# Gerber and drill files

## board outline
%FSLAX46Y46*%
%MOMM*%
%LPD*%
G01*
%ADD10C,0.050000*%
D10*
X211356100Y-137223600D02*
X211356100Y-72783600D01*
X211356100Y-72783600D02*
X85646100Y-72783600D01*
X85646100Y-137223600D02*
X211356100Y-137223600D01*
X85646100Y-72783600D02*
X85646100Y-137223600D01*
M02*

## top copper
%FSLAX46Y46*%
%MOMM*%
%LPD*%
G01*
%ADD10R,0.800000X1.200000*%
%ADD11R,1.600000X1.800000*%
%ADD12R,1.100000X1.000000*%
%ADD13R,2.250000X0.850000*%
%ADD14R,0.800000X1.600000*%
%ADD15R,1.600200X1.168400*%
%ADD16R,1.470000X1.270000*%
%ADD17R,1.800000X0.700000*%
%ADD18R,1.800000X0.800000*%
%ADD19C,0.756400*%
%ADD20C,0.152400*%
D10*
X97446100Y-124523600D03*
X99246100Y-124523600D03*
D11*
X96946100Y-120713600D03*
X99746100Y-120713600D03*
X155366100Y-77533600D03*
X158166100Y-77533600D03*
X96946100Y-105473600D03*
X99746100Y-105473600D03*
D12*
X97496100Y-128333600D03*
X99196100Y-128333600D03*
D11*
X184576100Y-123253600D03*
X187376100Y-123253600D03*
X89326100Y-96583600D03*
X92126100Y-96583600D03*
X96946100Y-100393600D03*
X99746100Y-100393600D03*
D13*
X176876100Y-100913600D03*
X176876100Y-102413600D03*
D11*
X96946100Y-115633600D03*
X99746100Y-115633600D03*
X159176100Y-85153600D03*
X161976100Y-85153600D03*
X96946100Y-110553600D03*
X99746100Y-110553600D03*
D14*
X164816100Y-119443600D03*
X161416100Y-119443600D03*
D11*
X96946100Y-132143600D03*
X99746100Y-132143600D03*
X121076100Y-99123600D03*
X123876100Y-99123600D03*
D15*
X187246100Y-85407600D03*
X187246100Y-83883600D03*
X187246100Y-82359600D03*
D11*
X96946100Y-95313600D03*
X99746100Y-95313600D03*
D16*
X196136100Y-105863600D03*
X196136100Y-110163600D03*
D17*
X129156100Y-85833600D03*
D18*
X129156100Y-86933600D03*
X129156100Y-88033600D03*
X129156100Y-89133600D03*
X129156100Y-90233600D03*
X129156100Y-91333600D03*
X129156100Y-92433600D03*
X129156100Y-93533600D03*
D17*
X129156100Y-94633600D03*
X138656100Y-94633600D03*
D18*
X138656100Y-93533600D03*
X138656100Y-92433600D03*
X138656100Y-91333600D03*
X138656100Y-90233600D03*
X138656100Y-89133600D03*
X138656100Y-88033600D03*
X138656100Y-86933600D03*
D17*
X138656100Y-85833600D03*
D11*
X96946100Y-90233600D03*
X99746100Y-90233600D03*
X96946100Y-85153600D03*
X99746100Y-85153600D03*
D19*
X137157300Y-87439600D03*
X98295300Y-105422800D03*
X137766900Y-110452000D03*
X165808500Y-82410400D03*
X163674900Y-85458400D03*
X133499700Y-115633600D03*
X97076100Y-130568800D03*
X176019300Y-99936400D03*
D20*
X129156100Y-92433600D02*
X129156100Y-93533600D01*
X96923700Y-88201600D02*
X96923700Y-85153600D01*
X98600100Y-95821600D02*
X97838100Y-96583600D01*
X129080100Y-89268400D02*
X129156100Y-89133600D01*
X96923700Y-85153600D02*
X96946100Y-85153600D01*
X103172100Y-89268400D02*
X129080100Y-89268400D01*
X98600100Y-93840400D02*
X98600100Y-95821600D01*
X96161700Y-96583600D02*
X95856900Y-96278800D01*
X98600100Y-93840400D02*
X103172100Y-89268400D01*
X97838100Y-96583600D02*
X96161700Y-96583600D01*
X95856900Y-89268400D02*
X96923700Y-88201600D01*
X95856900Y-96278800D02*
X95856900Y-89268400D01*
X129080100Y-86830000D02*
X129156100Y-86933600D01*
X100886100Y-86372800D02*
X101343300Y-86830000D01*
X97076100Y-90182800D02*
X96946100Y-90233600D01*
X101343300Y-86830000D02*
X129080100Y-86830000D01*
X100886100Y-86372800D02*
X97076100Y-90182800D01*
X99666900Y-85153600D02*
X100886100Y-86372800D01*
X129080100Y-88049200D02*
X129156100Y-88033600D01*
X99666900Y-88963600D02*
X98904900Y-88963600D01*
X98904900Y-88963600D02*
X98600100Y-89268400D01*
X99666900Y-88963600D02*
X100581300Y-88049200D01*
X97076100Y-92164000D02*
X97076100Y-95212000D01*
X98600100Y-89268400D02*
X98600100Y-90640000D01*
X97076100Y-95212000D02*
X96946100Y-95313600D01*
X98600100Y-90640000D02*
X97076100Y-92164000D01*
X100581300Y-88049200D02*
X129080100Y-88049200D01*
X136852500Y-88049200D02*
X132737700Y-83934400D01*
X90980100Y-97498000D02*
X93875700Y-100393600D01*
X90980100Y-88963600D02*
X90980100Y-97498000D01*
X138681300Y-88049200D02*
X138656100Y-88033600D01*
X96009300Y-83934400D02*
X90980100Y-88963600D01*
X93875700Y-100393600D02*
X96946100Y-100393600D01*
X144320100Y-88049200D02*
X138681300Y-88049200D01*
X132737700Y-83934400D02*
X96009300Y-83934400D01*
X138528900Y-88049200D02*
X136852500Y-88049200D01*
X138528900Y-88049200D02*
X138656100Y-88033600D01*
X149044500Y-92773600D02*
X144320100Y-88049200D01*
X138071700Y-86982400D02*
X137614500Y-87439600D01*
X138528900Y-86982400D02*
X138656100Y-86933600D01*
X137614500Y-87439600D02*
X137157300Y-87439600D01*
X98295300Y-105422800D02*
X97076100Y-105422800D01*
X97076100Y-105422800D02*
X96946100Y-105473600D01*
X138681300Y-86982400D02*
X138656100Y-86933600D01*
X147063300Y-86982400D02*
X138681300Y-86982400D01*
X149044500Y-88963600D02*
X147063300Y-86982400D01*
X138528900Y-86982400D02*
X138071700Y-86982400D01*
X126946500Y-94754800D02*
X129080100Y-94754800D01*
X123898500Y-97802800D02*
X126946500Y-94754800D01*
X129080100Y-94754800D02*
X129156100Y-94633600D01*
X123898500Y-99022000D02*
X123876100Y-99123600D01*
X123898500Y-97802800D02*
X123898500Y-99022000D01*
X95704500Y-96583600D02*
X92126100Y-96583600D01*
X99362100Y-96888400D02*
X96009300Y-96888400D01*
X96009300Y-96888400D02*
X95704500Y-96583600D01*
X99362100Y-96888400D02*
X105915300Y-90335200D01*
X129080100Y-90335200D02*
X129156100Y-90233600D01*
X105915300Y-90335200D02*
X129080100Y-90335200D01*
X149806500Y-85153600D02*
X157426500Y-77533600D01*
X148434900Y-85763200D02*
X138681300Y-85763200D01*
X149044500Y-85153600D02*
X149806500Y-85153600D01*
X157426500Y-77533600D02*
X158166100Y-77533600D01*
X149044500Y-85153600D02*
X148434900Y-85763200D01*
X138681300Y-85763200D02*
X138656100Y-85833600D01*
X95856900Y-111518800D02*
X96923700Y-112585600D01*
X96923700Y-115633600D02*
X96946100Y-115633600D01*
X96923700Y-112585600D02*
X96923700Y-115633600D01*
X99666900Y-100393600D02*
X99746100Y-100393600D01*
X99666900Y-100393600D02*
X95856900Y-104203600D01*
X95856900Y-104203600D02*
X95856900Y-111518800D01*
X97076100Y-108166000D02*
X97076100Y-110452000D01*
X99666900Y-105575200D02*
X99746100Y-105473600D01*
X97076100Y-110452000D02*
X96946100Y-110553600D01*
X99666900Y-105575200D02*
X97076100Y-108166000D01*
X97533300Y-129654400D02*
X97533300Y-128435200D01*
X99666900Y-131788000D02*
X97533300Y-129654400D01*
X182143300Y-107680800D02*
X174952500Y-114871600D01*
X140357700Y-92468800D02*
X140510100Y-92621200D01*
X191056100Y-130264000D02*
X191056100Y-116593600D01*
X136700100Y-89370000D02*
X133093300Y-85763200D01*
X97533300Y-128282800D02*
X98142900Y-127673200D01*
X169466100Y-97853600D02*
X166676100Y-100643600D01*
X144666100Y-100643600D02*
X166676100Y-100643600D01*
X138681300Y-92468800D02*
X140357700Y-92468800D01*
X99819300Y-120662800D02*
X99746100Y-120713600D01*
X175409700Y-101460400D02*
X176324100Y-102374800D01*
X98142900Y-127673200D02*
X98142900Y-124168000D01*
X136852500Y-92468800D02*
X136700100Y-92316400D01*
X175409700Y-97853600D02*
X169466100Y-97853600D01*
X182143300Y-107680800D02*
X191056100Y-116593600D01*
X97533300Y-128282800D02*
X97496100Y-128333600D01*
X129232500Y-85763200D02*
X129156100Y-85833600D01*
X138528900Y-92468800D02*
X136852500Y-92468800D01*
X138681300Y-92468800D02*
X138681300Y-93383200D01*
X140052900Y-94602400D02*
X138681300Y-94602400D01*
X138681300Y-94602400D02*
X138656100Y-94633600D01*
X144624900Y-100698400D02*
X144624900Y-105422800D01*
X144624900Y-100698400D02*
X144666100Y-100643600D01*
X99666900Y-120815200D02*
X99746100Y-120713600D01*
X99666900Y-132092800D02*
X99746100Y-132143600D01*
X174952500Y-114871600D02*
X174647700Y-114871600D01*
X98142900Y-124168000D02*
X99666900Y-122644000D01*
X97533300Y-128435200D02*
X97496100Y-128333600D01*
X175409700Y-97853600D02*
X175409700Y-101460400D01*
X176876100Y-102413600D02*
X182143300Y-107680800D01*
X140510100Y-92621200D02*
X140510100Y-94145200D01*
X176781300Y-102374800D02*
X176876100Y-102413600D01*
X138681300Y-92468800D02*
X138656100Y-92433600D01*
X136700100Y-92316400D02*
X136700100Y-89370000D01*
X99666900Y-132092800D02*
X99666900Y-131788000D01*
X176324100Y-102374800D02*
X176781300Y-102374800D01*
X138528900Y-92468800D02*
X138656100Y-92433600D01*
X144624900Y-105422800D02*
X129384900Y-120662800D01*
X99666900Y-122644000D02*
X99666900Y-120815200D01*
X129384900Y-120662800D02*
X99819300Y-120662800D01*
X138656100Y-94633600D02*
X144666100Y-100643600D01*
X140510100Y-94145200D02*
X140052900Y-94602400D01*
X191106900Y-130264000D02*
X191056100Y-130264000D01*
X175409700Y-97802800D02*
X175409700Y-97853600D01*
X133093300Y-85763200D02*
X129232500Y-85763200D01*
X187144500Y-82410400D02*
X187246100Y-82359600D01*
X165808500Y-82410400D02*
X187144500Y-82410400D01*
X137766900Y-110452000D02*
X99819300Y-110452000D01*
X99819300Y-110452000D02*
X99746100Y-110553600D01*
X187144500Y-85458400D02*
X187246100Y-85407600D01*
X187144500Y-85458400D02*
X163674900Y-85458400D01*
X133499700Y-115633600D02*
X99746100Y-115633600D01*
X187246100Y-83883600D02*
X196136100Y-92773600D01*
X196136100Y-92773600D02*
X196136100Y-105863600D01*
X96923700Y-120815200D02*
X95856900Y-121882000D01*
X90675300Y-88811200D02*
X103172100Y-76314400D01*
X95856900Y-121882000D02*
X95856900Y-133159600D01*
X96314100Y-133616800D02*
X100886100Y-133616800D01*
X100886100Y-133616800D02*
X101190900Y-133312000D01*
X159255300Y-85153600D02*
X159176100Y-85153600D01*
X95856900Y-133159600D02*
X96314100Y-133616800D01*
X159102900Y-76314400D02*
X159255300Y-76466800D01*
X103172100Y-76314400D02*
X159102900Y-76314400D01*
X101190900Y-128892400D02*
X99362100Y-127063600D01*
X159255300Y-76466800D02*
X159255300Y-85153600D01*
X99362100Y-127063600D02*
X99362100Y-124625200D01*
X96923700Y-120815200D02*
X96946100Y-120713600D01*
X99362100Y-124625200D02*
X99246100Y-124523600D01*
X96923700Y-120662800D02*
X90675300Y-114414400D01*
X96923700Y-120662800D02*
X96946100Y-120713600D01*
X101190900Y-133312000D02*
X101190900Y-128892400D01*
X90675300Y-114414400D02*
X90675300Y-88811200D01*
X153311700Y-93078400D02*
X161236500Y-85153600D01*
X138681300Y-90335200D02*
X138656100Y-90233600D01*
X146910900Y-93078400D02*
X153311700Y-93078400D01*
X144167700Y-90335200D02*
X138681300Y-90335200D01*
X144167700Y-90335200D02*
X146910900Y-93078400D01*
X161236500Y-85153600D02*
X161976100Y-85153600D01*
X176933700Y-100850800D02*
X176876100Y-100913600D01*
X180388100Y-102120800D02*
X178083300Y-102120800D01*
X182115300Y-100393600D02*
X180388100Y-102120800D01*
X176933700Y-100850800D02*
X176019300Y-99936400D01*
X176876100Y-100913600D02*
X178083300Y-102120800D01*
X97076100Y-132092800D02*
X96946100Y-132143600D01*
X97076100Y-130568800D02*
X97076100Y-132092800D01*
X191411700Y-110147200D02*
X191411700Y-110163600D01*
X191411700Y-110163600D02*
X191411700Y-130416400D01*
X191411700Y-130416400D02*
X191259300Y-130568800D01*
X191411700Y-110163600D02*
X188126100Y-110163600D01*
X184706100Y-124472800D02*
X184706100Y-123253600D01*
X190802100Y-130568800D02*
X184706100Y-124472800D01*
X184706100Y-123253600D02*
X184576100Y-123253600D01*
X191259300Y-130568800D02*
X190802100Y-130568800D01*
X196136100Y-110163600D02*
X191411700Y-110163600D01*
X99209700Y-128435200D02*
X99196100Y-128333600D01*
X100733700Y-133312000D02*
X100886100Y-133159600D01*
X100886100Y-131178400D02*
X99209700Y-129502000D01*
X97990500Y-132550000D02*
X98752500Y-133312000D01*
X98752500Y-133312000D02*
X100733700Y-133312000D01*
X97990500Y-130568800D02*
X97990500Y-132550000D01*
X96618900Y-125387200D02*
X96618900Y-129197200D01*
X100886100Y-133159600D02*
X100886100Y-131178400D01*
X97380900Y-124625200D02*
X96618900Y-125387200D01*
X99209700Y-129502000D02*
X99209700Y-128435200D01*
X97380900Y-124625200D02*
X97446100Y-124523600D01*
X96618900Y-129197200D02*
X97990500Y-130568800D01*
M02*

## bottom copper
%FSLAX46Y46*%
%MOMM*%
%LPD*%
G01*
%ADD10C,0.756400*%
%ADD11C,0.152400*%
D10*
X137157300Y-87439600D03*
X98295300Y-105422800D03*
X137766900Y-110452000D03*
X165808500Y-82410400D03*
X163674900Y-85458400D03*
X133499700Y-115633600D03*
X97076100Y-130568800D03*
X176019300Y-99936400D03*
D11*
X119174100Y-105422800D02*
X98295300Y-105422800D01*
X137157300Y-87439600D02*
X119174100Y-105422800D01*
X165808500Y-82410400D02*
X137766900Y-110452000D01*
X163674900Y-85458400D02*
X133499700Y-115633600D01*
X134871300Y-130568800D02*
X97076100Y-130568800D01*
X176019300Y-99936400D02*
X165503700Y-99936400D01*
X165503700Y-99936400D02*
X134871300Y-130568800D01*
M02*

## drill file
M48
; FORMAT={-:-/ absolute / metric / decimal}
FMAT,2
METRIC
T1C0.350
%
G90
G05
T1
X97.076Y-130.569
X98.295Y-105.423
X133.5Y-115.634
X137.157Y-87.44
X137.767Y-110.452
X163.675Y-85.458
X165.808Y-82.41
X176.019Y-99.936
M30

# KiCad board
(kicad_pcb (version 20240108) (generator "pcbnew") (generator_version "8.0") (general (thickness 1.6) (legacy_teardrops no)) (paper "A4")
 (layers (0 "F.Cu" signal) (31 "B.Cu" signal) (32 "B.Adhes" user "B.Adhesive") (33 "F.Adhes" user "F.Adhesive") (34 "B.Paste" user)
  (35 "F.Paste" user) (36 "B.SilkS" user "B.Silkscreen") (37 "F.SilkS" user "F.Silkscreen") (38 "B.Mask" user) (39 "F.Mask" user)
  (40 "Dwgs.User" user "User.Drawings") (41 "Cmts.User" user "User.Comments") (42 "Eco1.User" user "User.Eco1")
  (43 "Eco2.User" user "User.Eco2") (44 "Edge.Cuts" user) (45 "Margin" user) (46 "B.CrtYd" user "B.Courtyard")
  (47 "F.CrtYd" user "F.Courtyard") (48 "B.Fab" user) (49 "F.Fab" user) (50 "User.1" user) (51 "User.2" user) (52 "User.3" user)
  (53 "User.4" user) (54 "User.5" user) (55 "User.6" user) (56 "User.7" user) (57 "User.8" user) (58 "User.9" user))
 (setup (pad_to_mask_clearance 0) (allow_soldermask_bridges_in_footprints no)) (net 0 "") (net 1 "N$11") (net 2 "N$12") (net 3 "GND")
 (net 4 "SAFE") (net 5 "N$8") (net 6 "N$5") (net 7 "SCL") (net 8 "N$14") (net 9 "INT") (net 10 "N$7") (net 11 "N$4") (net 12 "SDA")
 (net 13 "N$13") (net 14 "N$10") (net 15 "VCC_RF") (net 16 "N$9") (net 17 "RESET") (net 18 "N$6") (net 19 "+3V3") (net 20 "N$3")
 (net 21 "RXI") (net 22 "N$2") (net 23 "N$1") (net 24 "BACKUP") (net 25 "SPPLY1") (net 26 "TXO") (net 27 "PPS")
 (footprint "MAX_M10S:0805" (layer "F.Cu") (at 98.3461 124.5236)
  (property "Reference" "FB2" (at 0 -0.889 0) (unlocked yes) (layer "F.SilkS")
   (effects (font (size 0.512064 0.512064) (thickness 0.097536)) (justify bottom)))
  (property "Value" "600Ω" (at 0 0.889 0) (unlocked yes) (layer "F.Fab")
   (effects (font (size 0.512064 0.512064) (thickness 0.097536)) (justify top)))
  (pad "1" smd rect (at -0.9 0) (size 0.8 1.2) (layers "F.Cu" "F.Paste" "F.Mask") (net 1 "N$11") (solder_mask_margin 0.1016)
   (thermal_bridge_angle 0))
  (pad "2" smd rect (at 0.9 0) (size 0.8 1.2) (layers "F.Cu" "F.Paste" "F.Mask") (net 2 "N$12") (solder_mask_margin 0.1016)
   (thermal_bridge_angle 0)))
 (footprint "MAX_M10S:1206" (layer "F.Cu") (at 98.3461 120.7136)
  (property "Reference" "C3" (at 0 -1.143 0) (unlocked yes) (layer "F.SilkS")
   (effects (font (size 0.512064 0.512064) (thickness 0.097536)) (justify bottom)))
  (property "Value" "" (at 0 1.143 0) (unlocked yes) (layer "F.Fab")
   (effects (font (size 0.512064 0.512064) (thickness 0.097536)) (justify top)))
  (pad "1" smd rect (at -1.4 0) (size 1.6 1.8) (layers "F.Cu" "F.Paste" "F.Mask") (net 2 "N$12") (solder_mask_margin 0.1016)
   (thermal_bridge_angle 0))
  (pad "2" smd rect (at 1.4 0) (size 1.6 1.8) (layers "F.Cu" "F.Paste" "F.Mask") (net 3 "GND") (solder_mask_margin 0.1016)
   (thermal_bridge_angle 0)))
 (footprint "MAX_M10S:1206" (layer "F.Cu") (at 156.7661 77.5336)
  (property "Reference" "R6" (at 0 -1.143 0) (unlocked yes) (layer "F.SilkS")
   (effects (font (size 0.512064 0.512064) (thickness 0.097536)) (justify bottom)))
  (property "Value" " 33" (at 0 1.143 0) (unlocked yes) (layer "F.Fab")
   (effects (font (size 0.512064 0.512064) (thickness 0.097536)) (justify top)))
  (pad "1" smd rect (at -1.4 0) (size 1.6 1.8) (layers "F.Cu" "F.Paste" "F.Mask") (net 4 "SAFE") (solder_mask_margin 0.1016)
   (thermal_bridge_angle 0))
  (pad "2" smd rect (at 1.4 0) (size 1.6 1.8) (layers "F.Cu" "F.Paste" "F.Mask") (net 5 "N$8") (solder_mask_margin 0.1016)
   (thermal_bridge_angle 0)))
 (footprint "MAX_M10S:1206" (layer "F.Cu") (at 98.3461 105.4736)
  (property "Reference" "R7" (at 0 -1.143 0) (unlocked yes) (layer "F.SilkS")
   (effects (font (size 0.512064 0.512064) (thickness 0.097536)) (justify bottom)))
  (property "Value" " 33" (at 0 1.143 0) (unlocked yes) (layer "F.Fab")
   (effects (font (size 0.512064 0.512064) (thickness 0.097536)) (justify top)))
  (pad "1" smd rect (at -1.4 0) (size 1.6 1.8) (layers "F.Cu" "F.Paste" "F.Mask") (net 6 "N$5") (solder_mask_margin 0.1016)
   (thermal_bridge_angle 0))
  (pad "2" smd rect (at 1.4 0) (size 1.6 1.8) (layers "F.Cu" "F.Paste" "F.Mask") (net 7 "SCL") (solder_mask_margin 0.1016)
   (thermal_bridge_angle 0)))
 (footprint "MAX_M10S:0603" (layer "F.Cu") (at 98.3461 128.3336)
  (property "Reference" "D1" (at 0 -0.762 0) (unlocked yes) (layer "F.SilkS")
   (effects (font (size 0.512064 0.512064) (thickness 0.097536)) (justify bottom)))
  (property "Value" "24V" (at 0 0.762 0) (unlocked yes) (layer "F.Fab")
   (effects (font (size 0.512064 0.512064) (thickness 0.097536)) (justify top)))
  (pad "1" smd rect (at -0.85 0) (size 1.1 1) (layers "F.Cu" "F.Paste" "F.Mask") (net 3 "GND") (solder_mask_margin 0.1016)
   (thermal_bridge_angle 0))
  (pad "2" smd rect (at 0.85 0) (size 1.1 1) (layers "F.Cu" "F.Paste" "F.Mask") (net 1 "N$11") (solder_mask_margin 0.1016)
   (thermal_bridge_angle 0)))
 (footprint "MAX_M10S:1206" (layer "F.Cu") (at 185.9761 123.2536)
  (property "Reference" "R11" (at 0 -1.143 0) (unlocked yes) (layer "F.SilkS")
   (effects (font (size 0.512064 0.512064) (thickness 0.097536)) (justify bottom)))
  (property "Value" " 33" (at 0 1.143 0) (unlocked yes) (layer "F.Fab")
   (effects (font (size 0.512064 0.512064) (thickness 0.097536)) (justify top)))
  (pad "1" smd rect (at -1.4 0) (size 1.6 1.8) (layers "F.Cu" "F.Paste" "F.Mask") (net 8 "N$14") (solder_mask_margin 0.1016)
   (thermal_bridge_angle 0))
  (pad "2" smd rect (at 1.4 0) (size 1.6 1.8) (layers "F.Cu" "F.Paste" "F.Mask") (solder_mask_margin 0.1016) (thermal_bridge_angle 0)))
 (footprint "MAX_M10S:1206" (layer "F.Cu") (at 90.7261 96.5836)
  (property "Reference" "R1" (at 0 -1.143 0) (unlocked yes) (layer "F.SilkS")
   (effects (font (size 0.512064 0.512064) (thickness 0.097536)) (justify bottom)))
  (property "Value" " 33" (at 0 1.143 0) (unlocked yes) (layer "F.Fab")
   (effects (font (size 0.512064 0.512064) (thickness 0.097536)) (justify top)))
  (pad "1" smd rect (at -1.4 0) (size 1.6 1.8) (layers "F.Cu" "F.Paste" "F.Mask") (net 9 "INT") (solder_mask_margin 0.1016)
   (thermal_bridge_angle 0))
  (pad "2" smd rect (at 1.4 0) (size 1.6 1.8) (layers "F.Cu" "F.Paste" "F.Mask") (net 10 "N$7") (solder_mask_margin 0.1016)
   (thermal_bridge_angle 0)))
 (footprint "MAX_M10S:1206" (layer "F.Cu") (at 98.3461 100.3936)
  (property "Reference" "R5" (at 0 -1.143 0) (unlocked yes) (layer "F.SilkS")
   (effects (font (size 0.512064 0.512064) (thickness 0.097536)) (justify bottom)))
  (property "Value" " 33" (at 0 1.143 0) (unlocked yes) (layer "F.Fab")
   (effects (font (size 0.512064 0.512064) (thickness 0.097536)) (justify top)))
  (pad "1" smd rect (at -1.4 0) (size 1.6 1.8) (layers "F.Cu" "F.Paste" "F.Mask") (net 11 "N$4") (solder_mask_margin 0.1016)
   (thermal_bridge_angle 0))
  (pad "2" smd rect (at 1.4 0) (size 1.6 1.8) (layers "F.Cu" "F.Paste" "F.Mask") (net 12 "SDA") (solder_mask_margin 0.1016)
   (thermal_bridge_angle 0)))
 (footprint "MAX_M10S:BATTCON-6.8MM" (layer "F.Cu") (at 172.0061 101.6636)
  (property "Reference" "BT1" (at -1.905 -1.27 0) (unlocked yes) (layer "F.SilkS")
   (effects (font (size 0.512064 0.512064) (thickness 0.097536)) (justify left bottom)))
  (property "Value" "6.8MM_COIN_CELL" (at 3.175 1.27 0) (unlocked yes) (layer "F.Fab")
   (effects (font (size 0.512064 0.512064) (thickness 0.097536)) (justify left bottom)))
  (pad "+" smd rect (at 4.87 -0.75 180) (size 2.25 0.85) (layers "F.Cu" "F.Paste" "F.Mask") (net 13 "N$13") (solder_mask_margin 0.1016)
   (thermal_bridge_angle 0))
  (pad "-" smd rect (at 4.87 0.75 180) (size 2.25 0.85) (layers "F.Cu" "F.Paste" "F.Mask") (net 3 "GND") (solder_mask_margin 0.1016)
   (thermal_bridge_angle 0)))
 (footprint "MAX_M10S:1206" (layer "F.Cu") (at 98.3461 115.6336)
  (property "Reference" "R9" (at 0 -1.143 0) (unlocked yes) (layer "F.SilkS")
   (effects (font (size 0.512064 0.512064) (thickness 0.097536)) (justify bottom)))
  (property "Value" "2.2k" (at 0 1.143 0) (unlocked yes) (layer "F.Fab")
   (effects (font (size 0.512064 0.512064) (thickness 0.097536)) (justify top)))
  (pad "1" smd rect (at -1.4 0) (size 1.6 1.8) (layers "F.Cu" "F.Paste" "F.Mask") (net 12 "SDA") (solder_mask_margin 0.1016)
   (thermal_bridge_angle 0))
  (pad "2" smd rect (at 1.4 0) (size 1.6 1.8) (layers "F.Cu" "F.Paste" "F.Mask") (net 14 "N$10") (solder_mask_margin 0.1016)
   (thermal_bridge_angle 0)))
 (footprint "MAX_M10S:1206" (layer "F.Cu") (at 160.5761 85.1536)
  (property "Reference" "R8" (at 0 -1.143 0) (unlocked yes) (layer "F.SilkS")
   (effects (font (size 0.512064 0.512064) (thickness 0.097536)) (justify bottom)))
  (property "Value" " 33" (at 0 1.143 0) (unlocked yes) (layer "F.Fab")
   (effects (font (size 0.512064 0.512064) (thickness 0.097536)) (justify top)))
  (pad "1" smd rect (at -1.4 0) (size 1.6 1.8) (layers "F.Cu" "F.Paste" "F.Mask") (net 2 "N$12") (solder_mask_margin 0.1016)
   (thermal_bridge_angle 0))
  (pad "2" smd rect (at 1.4 0) (size 1.6 1.8) (layers "F.Cu" "F.Paste" "F.Mask") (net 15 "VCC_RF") (solder_mask_margin 0.1016)
   (thermal_bridge_angle 0)))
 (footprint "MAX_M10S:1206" (layer "F.Cu") (at 98.3461 110.5536)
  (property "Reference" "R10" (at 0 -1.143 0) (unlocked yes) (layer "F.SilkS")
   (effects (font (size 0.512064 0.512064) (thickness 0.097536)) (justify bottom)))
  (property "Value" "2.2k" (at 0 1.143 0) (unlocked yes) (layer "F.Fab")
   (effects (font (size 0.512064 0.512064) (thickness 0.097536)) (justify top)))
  (pad "1" smd rect (at -1.4 0) (size 1.6 1.8) (layers "F.Cu" "F.Paste" "F.Mask") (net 7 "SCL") (solder_mask_margin 0.1016)
   (thermal_bridge_angle 0))
  (pad "2" smd rect (at 1.4 0) (size 1.6 1.8) (layers "F.Cu" "F.Paste" "F.Mask") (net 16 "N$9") (solder_mask_margin 0.1016)
   (thermal_bridge_angle 0)))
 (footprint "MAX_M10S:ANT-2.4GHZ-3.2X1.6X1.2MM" (layer "F.Cu") (at 163.1161 119.4436 180)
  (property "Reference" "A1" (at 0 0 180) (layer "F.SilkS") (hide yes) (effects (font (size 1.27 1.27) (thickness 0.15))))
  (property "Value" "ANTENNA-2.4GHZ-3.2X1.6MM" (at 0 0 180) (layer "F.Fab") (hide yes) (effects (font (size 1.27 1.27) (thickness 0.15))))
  (pad "FEED" smd rect (at -1.7 0 180) (size 0.8 1.6) (layers "F.Cu" "F.Paste" "F.Mask") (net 1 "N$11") (solder_mask_margin 0.1016)
   (thermal_bridge_angle 0))
  (pad "NC" smd rect (at 1.7 0 180) (size 0.8 1.6) (layers "F.Cu" "F.Paste" "F.Mask") (solder_mask_margin 0.1016) (thermal_bridge_angle 0))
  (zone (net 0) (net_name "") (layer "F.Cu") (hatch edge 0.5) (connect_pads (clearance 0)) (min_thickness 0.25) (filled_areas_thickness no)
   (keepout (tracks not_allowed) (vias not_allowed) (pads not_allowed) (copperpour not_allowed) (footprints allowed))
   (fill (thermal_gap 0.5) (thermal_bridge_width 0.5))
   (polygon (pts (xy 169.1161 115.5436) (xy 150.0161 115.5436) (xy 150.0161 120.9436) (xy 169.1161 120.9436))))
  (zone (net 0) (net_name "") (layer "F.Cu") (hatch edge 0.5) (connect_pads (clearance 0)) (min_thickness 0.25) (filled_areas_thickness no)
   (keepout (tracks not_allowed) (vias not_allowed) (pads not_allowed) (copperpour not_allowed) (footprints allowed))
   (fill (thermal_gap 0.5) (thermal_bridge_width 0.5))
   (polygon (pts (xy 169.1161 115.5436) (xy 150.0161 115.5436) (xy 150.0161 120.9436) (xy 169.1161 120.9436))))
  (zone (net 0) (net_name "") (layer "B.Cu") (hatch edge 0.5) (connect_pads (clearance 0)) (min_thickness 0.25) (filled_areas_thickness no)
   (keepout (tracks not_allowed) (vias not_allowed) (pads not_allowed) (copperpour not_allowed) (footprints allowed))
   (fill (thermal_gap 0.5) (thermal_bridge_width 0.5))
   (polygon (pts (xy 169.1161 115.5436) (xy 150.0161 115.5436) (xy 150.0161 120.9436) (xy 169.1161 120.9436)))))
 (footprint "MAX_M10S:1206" (layer "F.Cu") (at 98.3461 132.1436)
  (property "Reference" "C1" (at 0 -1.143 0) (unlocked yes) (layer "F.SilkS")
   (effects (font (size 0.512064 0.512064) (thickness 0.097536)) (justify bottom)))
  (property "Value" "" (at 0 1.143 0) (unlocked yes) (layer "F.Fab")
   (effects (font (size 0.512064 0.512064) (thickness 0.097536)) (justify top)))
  (pad "1" smd rect (at -1.4 0) (size 1.6 1.8) (layers "F.Cu" "F.Paste" "F.Mask") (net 13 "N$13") (solder_mask_margin 0.1016)
   (thermal_bridge_angle 0))
  (pad "2" smd rect (at 1.4 0) (size 1.6 1.8) (layers "F.Cu" "F.Paste" "F.Mask") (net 3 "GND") (solder_mask_margin 0.1016)
   (thermal_bridge_angle 0)))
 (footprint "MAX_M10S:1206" (layer "F.Cu") (at 122.4761 99.1236)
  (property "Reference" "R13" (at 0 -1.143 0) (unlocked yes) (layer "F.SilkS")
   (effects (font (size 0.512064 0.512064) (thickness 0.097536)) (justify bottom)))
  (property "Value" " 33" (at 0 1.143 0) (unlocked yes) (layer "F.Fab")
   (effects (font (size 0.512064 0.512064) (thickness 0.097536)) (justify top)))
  (pad "1" smd rect (at -1.4 0) (size 1.6 1.8) (layers "F.Cu" "F.Paste" "F.Mask") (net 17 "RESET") (solder_mask_margin 0.1016)
   (thermal_bridge_angle 0))
  (pad "2" smd rect (at 1.4 0) (size 1.6 1.8) (layers "F.Cu" "F.Paste" "F.Mask") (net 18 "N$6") (solder_mask_margin 0.1016)
   (thermal_bridge_angle 0)))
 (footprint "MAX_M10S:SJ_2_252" (layer "F.Cu") (at 187.2461 83.8836 90)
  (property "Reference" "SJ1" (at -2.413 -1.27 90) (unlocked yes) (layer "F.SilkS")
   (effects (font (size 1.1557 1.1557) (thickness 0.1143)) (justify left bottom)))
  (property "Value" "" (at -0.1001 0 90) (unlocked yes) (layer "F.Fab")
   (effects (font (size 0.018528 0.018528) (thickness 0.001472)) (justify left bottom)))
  (pad "1" smd rect (at -1.524 0 90) (size 1.1684 1.6002) (layers "F.Cu" "F.Paste" "F.Mask") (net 14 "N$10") (solder_mask_margin 0.1016)
   (thermal_bridge_angle 0))
  (pad "2" smd rect (at 0 0 90) (size 1.1684 1.6002) (layers "F.Cu" "F.Paste" "F.Mask") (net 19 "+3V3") (solder_mask_margin 0.1016)
   (thermal_bridge_angle 0))
  (pad "3" smd rect (at 1.524 0 90) (size 1.1684 1.6002) (layers "F.Cu" "F.Paste" "F.Mask") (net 16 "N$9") (solder_mask_margin 0.1016)
   (thermal_bridge_angle 0)))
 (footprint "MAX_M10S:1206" (layer "F.Cu") (at 98.3461 95.3136)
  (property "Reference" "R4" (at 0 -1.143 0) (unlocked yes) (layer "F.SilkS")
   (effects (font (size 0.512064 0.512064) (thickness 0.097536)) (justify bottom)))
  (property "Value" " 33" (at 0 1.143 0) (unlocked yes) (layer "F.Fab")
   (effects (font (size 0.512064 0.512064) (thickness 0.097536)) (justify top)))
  (pad "1" smd rect (at -1.4 0) (size 1.6 1.8) (layers "F.Cu" "F.Paste" "F.Mask") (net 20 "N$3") (solder_mask_margin 0.1016)
   (thermal_bridge_angle 0))
  (pad "2" smd rect (at 1.4 0) (size 1.6 1.8) (layers "F.Cu" "F.Paste" "F.Mask") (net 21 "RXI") (solder_mask_margin 0.1016)
   (thermal_bridge_angle 0)))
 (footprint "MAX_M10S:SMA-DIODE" (layer "F.Cu") (at 196.1361 108.0136 -90)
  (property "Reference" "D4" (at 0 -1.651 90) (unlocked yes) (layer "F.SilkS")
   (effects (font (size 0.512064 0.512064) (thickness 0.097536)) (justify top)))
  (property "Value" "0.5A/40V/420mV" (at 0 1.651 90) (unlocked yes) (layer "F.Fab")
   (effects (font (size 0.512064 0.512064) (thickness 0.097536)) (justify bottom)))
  (pad "A" smd rect (at -2.15 0 90) (size 1.27 1.47) (layers "F.Cu" "F.Paste" "F.Mask") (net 19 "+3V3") (solder_mask_margin 0.1016)
   (thermal_bridge_angle 0))
  (pad "C" smd rect (at 2.15 0 270) (size 1.27 1.47) (layers "F.Cu" "F.Paste" "F.Mask") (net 8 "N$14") (solder_mask_margin 0.1016)
   (thermal_bridge_angle 0)))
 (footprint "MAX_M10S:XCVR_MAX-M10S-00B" (layer "F.Cu") (at 133.9061 90.2336)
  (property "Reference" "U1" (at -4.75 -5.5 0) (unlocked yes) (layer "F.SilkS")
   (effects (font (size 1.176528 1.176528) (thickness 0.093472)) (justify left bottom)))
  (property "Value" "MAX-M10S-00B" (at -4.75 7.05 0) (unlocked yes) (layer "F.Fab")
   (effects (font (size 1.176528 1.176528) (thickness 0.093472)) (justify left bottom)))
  (pad "1" smd rect (at -4.75 -4.4) (size 1.8 0.7) (layers "F.Cu" "F.Mask") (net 3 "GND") (solder_mask_margin 0.1016)
   (thermal_bridge_angle 0))
  (pad "2" smd rect (at -4.75 -3.3) (size 1.8 0.8) (layers "F.Cu" "F.Mask") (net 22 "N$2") (solder_mask_margin 0.1016)
   (thermal_bridge_angle 0))
  (pad "3" smd rect (at -4.75 -2.2) (size 1.8 0.8) (layers "F.Cu" "F.Mask") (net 20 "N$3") (solder_mask_margin 0.1016)
   (thermal_bridge_angle 0))
  (pad "4" smd rect (at -4.75 -1.1) (size 1.8 0.8) (layers "F.Cu" "F.Mask") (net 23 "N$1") (solder_mask_margin 0.1016)
   (thermal_bridge_angle 0))
  (pad "5" smd rect (at -4.75 0) (size 1.8 0.8) (layers "F.Cu" "F.Mask") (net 10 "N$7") (solder_mask_margin 0.1016) (thermal_bridge_angle 0))
  (pad "6" smd rect (at -4.75 1.1) (size 1.8 0.8) (layers "F.Cu" "F.Mask") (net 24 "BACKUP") (solder_mask_margin 0.1016)
   (thermal_bridge_angle 0))
  (pad "7" smd rect (at -4.75 2.2) (size 1.8 0.8) (layers "F.Cu" "F.Mask") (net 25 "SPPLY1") (solder_mask_margin 0.1016)
   (thermal_bridge_angle 0))
  (pad "8" smd rect (at -4.75 3.3) (size 1.8 0.8) (layers "F.Cu" "F.Mask") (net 25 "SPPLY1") (solder_mask_margin 0.1016)
   (thermal_bridge_angle 0))
  (pad "9" smd rect (at -4.75 4.4) (size 1.8 0.7) (layers "F.Cu" "F.Mask") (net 18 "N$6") (solder_mask_margin 0.1016)
   (thermal_bridge_angle 0))
  (pad "10" smd rect (at 4.75 4.4) (size 1.8 0.7) (layers "F.Cu" "F.Mask") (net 3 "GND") (solder_mask_margin 0.1016)
   (thermal_bridge_angle 0))
  (pad "11" smd rect (at 4.75 3.3) (size 1.8 0.8) (layers "F.Cu" "F.Mask") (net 1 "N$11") (solder_mask_margin 0.1016)
   (thermal_bridge_angle 0))
  (pad "12" smd rect (at 4.75 2.2) (size 1.8 0.8) (layers "F.Cu" "F.Mask") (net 3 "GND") (solder_mask_margin 0.1016)
   (thermal_bridge_angle 0))
  (pad "13" smd rect (at 4.75 1.1) (size 1.8 0.8) (layers "F.Cu" "F.Mask") (solder_mask_margin 0.1016) (thermal_bridge_angle 0))
  (pad "14" smd rect (at 4.75 0) (size 1.8 0.8) (layers "F.Cu" "F.Mask") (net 15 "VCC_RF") (solder_mask_margin 0.1016)
   (thermal_bridge_angle 0))
  (pad "15" smd rect (at 4.75 -1.1) (size 1.8 0.8) (layers "F.Cu" "F.Mask") (solder_mask_margin 0.1016) (thermal_bridge_angle 0))
  (pad "16" smd rect (at 4.75 -2.2) (size 1.8 0.8) (layers "F.Cu" "F.Mask") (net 11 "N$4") (solder_mask_margin 0.1016)
   (thermal_bridge_angle 0))
  (pad "17" smd rect (at 4.75 -3.3) (size 1.8 0.8) (layers "F.Cu" "F.Mask") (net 6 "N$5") (solder_mask_margin 0.1016)
   (thermal_bridge_angle 0))
  (pad "18" smd rect (at 4.75 -4.4) (size 1.8 0.7) (layers "F.Cu" "F.Mask") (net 5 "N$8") (solder_mask_margin 0.1016)
   (thermal_bridge_angle 0))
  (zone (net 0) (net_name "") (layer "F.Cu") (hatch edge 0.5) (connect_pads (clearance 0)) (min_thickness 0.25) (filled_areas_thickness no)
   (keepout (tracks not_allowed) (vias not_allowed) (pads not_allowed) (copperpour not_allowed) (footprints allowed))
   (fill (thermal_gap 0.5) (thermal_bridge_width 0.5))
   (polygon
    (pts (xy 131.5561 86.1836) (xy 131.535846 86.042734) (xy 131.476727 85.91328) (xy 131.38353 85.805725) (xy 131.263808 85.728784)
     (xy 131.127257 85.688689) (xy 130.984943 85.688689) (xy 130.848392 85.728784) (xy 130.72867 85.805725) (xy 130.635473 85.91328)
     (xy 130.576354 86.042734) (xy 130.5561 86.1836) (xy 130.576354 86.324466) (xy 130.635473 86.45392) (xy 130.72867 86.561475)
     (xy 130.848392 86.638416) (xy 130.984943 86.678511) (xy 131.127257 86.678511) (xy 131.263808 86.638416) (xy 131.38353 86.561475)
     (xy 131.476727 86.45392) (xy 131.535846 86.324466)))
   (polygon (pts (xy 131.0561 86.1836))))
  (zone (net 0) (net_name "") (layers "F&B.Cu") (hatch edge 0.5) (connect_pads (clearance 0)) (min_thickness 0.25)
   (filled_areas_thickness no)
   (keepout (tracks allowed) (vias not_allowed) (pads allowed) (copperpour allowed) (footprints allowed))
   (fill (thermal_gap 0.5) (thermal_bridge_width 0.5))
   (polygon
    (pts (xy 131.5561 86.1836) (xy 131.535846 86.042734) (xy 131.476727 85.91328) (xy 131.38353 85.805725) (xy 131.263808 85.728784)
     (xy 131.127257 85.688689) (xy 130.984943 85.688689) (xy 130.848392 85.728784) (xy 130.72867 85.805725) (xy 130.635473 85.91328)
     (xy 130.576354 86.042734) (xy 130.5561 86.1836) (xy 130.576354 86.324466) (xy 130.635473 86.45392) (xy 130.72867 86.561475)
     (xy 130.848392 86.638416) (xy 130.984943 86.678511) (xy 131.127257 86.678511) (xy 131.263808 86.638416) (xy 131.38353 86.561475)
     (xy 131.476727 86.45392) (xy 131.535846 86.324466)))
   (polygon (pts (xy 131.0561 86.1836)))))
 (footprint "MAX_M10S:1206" (layer "F.Cu") (at 98.3461 90.2336)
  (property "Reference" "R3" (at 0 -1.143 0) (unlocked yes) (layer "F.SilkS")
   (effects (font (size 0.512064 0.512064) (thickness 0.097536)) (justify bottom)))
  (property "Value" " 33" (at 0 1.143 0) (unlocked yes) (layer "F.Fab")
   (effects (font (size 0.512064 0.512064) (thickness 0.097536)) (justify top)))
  (pad "1" smd rect (at -1.4 0) (size 1.6 1.8) (layers "F.Cu" "F.Paste" "F.Mask") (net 22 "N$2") (solder_mask_margin 0.1016)
   (thermal_bridge_angle 0))
  (pad "2" smd rect (at 1.4 0) (size 1.6 1.8) (layers "F.Cu" "F.Paste" "F.Mask") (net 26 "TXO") (solder_mask_margin 0.1016)
   (thermal_bridge_angle 0)))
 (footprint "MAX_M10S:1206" (layer "F.Cu") (at 98.3461 85.1536)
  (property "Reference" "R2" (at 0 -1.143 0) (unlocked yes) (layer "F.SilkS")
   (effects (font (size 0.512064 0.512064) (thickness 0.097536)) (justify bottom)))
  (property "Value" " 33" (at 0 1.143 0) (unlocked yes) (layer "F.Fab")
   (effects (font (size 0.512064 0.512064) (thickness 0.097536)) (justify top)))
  (pad "1" smd rect (at -1.4 0) (size 1.6 1.8) (layers "F.Cu" "F.Paste" "F.Mask") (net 23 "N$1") (solder_mask_margin 0.1016)
   (thermal_bridge_angle 0))
  (pad "2" smd rect (at 1.4 0) (size 1.6 1.8) (layers "F.Cu" "F.Paste" "F.Mask") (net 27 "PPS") (solder_mask_margin 0.1016)
   (thermal_bridge_angle 0)))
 (gr_line (start 211.3561 137.2236) (end 211.3561 72.7836) (stroke (width 0.05) (type solid)) (layer "Edge.Cuts"))
 (gr_line (start 211.3561 72.7836) (end 85.6461 72.7836) (stroke (width 0.05) (type solid)) (layer "Edge.Cuts"))
 (gr_line (start 85.6461 137.2236) (end 211.3561 137.2236) (stroke (width 0.05) (type solid)) (layer "Edge.Cuts"))
 (gr_line (start 85.6461 72.7836) (end 85.6461 137.2236) (stroke (width 0.05) (type solid)) (layer "Edge.Cuts"))
 (segment (start 129.1561 92.4336) (end 129.1561 93.5336) (width 0.1524) (layer "F.Cu") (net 25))
 (segment (start 96.9237 88.2016) (end 96.9237 85.1536) (width 0.1524) (layer "F.Cu") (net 23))
 (segment (start 98.6001 95.8216) (end 97.8381 96.5836) (width 0.1524) (layer "F.Cu") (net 23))
 (segment (start 129.0801 89.2684) (end 129.1561 89.1336) (width 0.1524) (layer "F.Cu") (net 23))
 (segment (start 96.9237 85.1536) (end 96.9461 85.1536) (width 0.1524) (layer "F.Cu") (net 23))
 (segment (start 103.1721 89.2684) (end 129.0801 89.2684) (width 0.1524) (layer "F.Cu") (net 23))
 (segment (start 98.6001 93.8404) (end 98.6001 95.8216) (width 0.1524) (layer "F.Cu") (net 23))
 (segment (start 96.1617 96.5836) (end 95.8569 96.2788) (width 0.1524) (layer "F.Cu") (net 23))
 (segment (start 98.6001 93.8404) (end 103.1721 89.2684) (width 0.1524) (layer "F.Cu") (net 23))
 (segment (start 97.8381 96.5836) (end 96.1617 96.5836) (width 0.1524) (layer "F.Cu") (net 23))
 (segment (start 95.8569 89.2684) (end 96.9237 88.2016) (width 0.1524) (layer "F.Cu") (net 23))
 (segment (start 95.8569 96.2788) (end 95.8569 89.2684) (width 0.1524) (layer "F.Cu") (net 23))
 (segment (start 129.0801 86.83) (end 129.1561 86.9336) (width 0.1524) (layer "F.Cu") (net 22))
 (segment (start 100.8861 86.3728) (end 101.3433 86.83) (width 0.1524) (layer "F.Cu") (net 22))
 (segment (start 97.0761 90.1828) (end 96.9461 90.2336) (width 0.1524) (layer "F.Cu") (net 22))
 (segment (start 101.3433 86.83) (end 129.0801 86.83) (width 0.1524) (layer "F.Cu") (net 22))
 (segment (start 100.8861 86.3728) (end 97.0761 90.1828) (width 0.1524) (layer "F.Cu") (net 22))
 (segment (start 99.6669 85.1536) (end 100.8861 86.3728) (width 0.1524) (layer "F.Cu") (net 22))
 (segment (start 129.0801 88.0492) (end 129.1561 88.0336) (width 0.1524) (layer "F.Cu") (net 20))
 (segment (start 99.6669 88.9636) (end 98.9049 88.9636) (width 0.1524) (layer "F.Cu") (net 20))
 (segment (start 98.9049 88.9636) (end 98.6001 89.2684) (width 0.1524) (layer "F.Cu") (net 20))
 (segment (start 99.6669 88.9636) (end 100.5813 88.0492) (width 0.1524) (layer "F.Cu") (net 20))
 (segment (start 97.0761 92.164) (end 97.0761 95.212) (width 0.1524) (layer "F.Cu") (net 20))
 (segment (start 98.6001 89.2684) (end 98.6001 90.64) (width 0.1524) (layer "F.Cu") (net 20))
 (segment (start 97.0761 95.212) (end 96.9461 95.3136) (width 0.1524) (layer "F.Cu") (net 20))
 (segment (start 98.6001 90.64) (end 97.0761 92.164) (width 0.1524) (layer "F.Cu") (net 20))
 (segment (start 100.5813 88.0492) (end 129.0801 88.0492) (width 0.1524) (layer "F.Cu") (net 20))
 (segment (start 136.8525 88.0492) (end 132.7377 83.9344) (width 0.1524) (layer "F.Cu") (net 11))
 (segment (start 90.9801 97.498) (end 93.8757 100.3936) (width 0.1524) (layer "F.Cu") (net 11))
 (segment (start 90.9801 88.9636) (end 90.9801 97.498) (width 0.1524) (layer "F.Cu") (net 11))
 (segment (start 138.6813 88.0492) (end 138.6561 88.0336) (width 0.1524) (layer "F.Cu") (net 11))
 (segment (start 96.0093 83.9344) (end 90.9801 88.9636) (width 0.1524) (layer "F.Cu") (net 11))
 (segment (start 93.8757 100.3936) (end 96.9461 100.3936) (width 0.1524) (layer "F.Cu") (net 11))
 (segment (start 144.3201 88.0492) (end 138.6813 88.0492) (width 0.1524) (layer "F.Cu") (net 11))
 (segment (start 132.7377 83.9344) (end 96.0093 83.9344) (width 0.1524) (layer "F.Cu") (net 11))
 (segment (start 138.5289 88.0492) (end 136.8525 88.0492) (width 0.1524) (layer "F.Cu") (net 11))
 (segment (start 138.5289 88.0492) (end 138.6561 88.0336) (width 0.1524) (layer "F.Cu") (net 11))
 (segment (start 149.0445 92.7736) (end 144.3201 88.0492) (width 0.1524) (layer "F.Cu") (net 11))
 (segment (start 138.0717 86.9824) (end 137.6145 87.4396) (width 0.1524) (layer "F.Cu") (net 6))
 (segment (start 138.5289 86.9824) (end 138.6561 86.9336) (width 0.1524) (layer "F.Cu") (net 6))
 (segment (start 137.6145 87.4396) (end 137.1573 87.4396) (width 0.1524) (layer "F.Cu") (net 6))
 (segment (start 98.2953 105.4228) (end 97.0761 105.4228) (width 0.1524) (layer "F.Cu") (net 6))
 (segment (start 97.0761 105.4228) (end 96.9461 105.4736) (width 0.1524) (layer "F.Cu") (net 6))
 (segment (start 138.6813 86.9824) (end 138.6561 86.9336) (width 0.1524) (layer "F.Cu") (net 6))
 (segment (start 147.0633 86.9824) (end 138.6813 86.9824) (width 0.1524) (layer "F.Cu") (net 6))
 (segment (start 149.0445 88.9636) (end 147.0633 86.9824) (width 0.1524) (layer "F.Cu") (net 6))
 (segment (start 138.5289 86.9824) (end 138.0717 86.9824) (width 0.1524) (layer "F.Cu") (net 6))
 (via (at 137.1573 87.4396) (size 0.7564) (drill 0.35) (layers "F.Cu" "B.Cu") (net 6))
 (via (at 98.2953 105.4228) (size 0.7564) (drill 0.35) (layers "F.Cu" "B.Cu") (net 6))
 (segment (start 119.1741 105.4228) (end 98.2953 105.4228) (width 0.1524) (layer "B.Cu") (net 6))
 (segment (start 137.1573 87.4396) (end 119.1741 105.4228) (width 0.1524) (layer "B.Cu") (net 6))
 (segment (start 126.9465 94.7548) (end 129.0801 94.7548) (width 0.1524) (layer "F.Cu") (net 18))
 (segment (start 123.8985 97.8028) (end 126.9465 94.7548) (width 0.1524) (layer "F.Cu") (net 18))
 (segment (start 129.0801 94.7548) (end 129.1561 94.6336) (width 0.1524) (layer "F.Cu") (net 18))
 (segment (start 123.8985 99.022) (end 123.8761 99.1236) (width 0.1524) (layer "F.Cu") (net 18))
 (segment (start 123.8985 97.8028) (end 123.8985 99.022) (width 0.1524) (layer "F.Cu") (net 18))
 (segment (start 95.7045 96.5836) (end 92.1261 96.5836) (width 0.1524) (layer "F.Cu") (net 10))
 (segment (start 99.3621 96.8884) (end 96.0093 96.8884) (width 0.1524) (layer "F.Cu") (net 10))
 (segment (start 96.0093 96.8884) (end 95.7045 96.5836) (width 0.1524) (layer "F.Cu") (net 10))
 (segment (start 99.3621 96.8884) (end 105.9153 90.3352) (width 0.1524) (layer "F.Cu") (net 10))
 (segment (start 129.0801 90.3352) (end 129.1561 90.2336) (width 0.1524) (layer "F.Cu") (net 10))
 (segment (start 105.9153 90.3352) (end 129.0801 90.3352) (width 0.1524) (layer "F.Cu") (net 10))
 (segment (start 149.8065 85.1536) (end 157.4265 77.5336) (width 0.1524) (layer "F.Cu") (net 5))
 (segment (start 148.4349 85.7632) (end 138.6813 85.7632) (width 0.1524) (layer "F.Cu") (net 5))
 (segment (start 149.0445 85.1536) (end 149.8065 85.1536) (width 0.1524) (layer "F.Cu") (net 5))
 (segment (start 157.4265 77.5336) (end 158.1661 77.5336) (width 0.1524) (layer "F.Cu") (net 5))
 (segment (start 149.0445 85.1536) (end 148.4349 85.7632) (width 0.1524) (layer "F.Cu") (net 5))
 (segment (start 138.6813 85.7632) (end 138.6561 85.8336) (width 0.1524) (layer "F.Cu") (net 5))
 (segment (start 95.8569 111.5188) (end 96.9237 112.5856) (width 0.1524) (layer "F.Cu") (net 12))
 (segment (start 96.9237 115.6336) (end 96.9461 115.6336) (width 0.1524) (layer "F.Cu") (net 12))
 (segment (start 96.9237 112.5856) (end 96.9237 115.6336) (width 0.1524) (layer "F.Cu") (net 12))
 (segment (start 99.6669 100.3936) (end 99.7461 100.3936) (width 0.1524) (layer "F.Cu") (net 12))
 (segment (start 99.6669 100.3936) (end 95.8569 104.2036) (width 0.1524) (layer "F.Cu") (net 12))
 (segment (start 95.8569 104.2036) (end 95.8569 111.5188) (width 0.1524) (layer "F.Cu") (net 12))
 (segment (start 97.0761 108.166) (end 97.0761 110.452) (width 0.1524) (layer "F.Cu") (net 7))
 (segment (start 99.6669 105.5752) (end 99.7461 105.4736) (width 0.1524) (layer "F.Cu") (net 7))
 (segment (start 97.0761 110.452) (end 96.9461 110.5536) (width 0.1524) (layer "F.Cu") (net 7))
 (segment (start 99.6669 105.5752) (end 97.0761 108.166) (width 0.1524) (layer "F.Cu") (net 7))
 (segment (start 97.5333 129.6544) (end 97.5333 128.4352) (width 0.1524) (layer "F.Cu") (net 3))
 (segment (start 99.6669 131.788) (end 97.5333 129.6544) (width 0.1524) (layer "F.Cu") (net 3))
 (segment (start 182.1433 107.6808) (end 174.9525 114.8716) (width 0.1524) (layer "F.Cu") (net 3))
 (segment (start 140.3577 92.4688) (end 140.5101 92.6212) (width 0.1524) (layer "F.Cu") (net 3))
 (segment (start 191.0561 130.264) (end 191.0561 116.5936) (width 0.1524) (layer "F.Cu") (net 3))
 (segment (start 136.7001 89.37) (end 133.0933 85.7632) (width 0.1524) (layer "F.Cu") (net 3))
 (segment (start 97.5333 128.2828) (end 98.1429 127.6732) (width 0.1524) (layer "F.Cu") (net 3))
 (segment (start 169.4661 97.8536) (end 166.6761 100.6436) (width 0.1524) (layer "F.Cu") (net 3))
 (segment (start 144.6661 100.6436) (end 166.6761 100.6436) (width 0.1524) (layer "F.Cu") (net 3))
 (segment (start 138.6813 92.4688) (end 140.3577 92.4688) (width 0.1524) (layer "F.Cu") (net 3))
 (segment (start 99.8193 120.6628) (end 99.7461 120.7136) (width 0.1524) (layer "F.Cu") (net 3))
 (segment (start 175.4097 101.4604) (end 176.3241 102.3748) (width 0.1524) (layer "F.Cu") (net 3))
 (segment (start 98.1429 127.6732) (end 98.1429 124.168) (width 0.1524) (layer "F.Cu") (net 3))
 (segment (start 136.8525 92.4688) (end 136.7001 92.3164) (width 0.1524) (layer "F.Cu") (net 3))
 (segment (start 175.4097 97.8536) (end 169.4661 97.8536) (width 0.1524) (layer "F.Cu") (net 3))
 (segment (start 182.1433 107.6808) (end 191.0561 116.5936) (width 0.1524) (layer "F.Cu") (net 3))
 (segment (start 97.5333 128.2828) (end 97.4961 128.3336) (width 0.1524) (layer "F.Cu") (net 3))
 (segment (start 129.2325 85.7632) (end 129.1561 85.8336) (width 0.1524) (layer "F.Cu") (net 3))
 (segment (start 138.5289 92.4688) (end 136.8525 92.4688) (width 0.1524) (layer "F.Cu") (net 3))
 (segment (start 138.6813 92.4688) (end 138.6813 93.3832) (width 0.1524) (layer "F.Cu") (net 3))
 (segment (start 140.0529 94.6024) (end 138.6813 94.6024) (width 0.1524) (layer "F.Cu") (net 3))
 (segment (start 138.6813 94.6024) (end 138.6561 94.6336) (width 0.1524) (layer "F.Cu") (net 3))
 (segment (start 144.6249 100.6984) (end 144.6249 105.4228) (width 0.1524) (layer "F.Cu") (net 3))
 (segment (start 144.6249 100.6984) (end 144.6661 100.6436) (width 0.1524) (layer "F.Cu") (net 3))
 (segment (start 99.6669 120.8152) (end 99.7461 120.7136) (width 0.1524) (layer "F.Cu") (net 3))
 (segment (start 99.6669 132.0928) (end 99.7461 132.1436) (width 0.1524) (layer "F.Cu") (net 3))
 (segment (start 174.9525 114.8716) (end 174.6477 114.8716) (width 0.1524) (layer "F.Cu") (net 3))
 (segment (start 98.1429 124.168) (end 99.6669 122.644) (width 0.1524) (layer "F.Cu") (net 3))
 (segment (start 97.5333 128.4352) (end 97.4961 128.3336) (width 0.1524) (layer "F.Cu") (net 3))
 (segment (start 175.4097 97.8536) (end 175.4097 101.4604) (width 0.1524) (layer "F.Cu") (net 3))
 (segment (start 176.8761 102.4136) (end 182.1433 107.6808) (width 0.1524) (layer "F.Cu") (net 3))
 (segment (start 140.5101 92.6212) (end 140.5101 94.1452) (width 0.1524) (layer "F.Cu") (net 3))
 (segment (start 176.7813 102.3748) (end 176.8761 102.4136) (width 0.1524) (layer "F.Cu") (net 3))
 (segment (start 138.6813 92.4688) (end 138.6561 92.4336) (width 0.1524) (layer "F.Cu") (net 3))
 (segment (start 136.7001 92.3164) (end 136.7001 89.37) (width 0.1524) (layer "F.Cu") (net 3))
 (segment (start 99.6669 132.0928) (end 99.6669 131.788) (width 0.1524) (layer "F.Cu") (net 3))
 (segment (start 176.3241 102.3748) (end 176.7813 102.3748) (width 0.1524) (layer "F.Cu") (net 3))
 (segment (start 138.5289 92.4688) (end 138.6561 92.4336) (width 0.1524) (layer "F.Cu") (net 3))
 (segment (start 144.6249 105.4228) (end 129.3849 120.6628) (width 0.1524) (layer "F.Cu") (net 3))
 (segment (start 99.6669 122.644) (end 99.6669 120.8152) (width 0.1524) (layer "F.Cu") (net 3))
 (segment (start 129.3849 120.6628) (end 99.8193 120.6628) (width 0.1524) (layer "F.Cu") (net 3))
 (segment (start 138.6561 94.6336) (end 144.6661 100.6436) (width 0.1524) (layer "F.Cu") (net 3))
 (segment (start 140.5101 94.1452) (end 140.0529 94.6024) (width 0.1524) (layer "F.Cu") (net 3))
 (segment (start 191.1069 130.264) (end 191.0561 130.264) (width 0.1524) (layer "F.Cu") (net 3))
 (segment (start 175.4097 97.8028) (end 175.4097 97.8536) (width 0.1524) (layer "F.Cu") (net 3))
 (segment (start 133.0933 85.7632) (end 129.2325 85.7632) (width 0.1524) (layer "F.Cu") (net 3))
 (segment (start 187.1445 82.4104) (end 187.2461 82.3596) (width 0.1524) (layer "F.Cu") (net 16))
 (segment (start 165.8085 82.4104) (end 187.1445 82.4104) (width 0.1524) (layer "F.Cu") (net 16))
 (segment (start 137.7669 110.452) (end 99.8193 110.452) (width 0.1524) (layer "F.Cu") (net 16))
 (segment (start 99.8193 110.452) (end 99.7461 110.5536) (width 0.1524) (layer "F.Cu") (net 16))
 (via (at 137.7669 110.452) (size 0.7564) (drill 0.35) (layers "F.Cu" "B.Cu") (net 16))
 (via (at 165.8085 82.4104) (size 0.7564) (drill 0.35) (layers "F.Cu" "B.Cu") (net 16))
 (segment (start 165.8085 82.4104) (end 137.7669 110.452) (width 0.1524) (layer "B.Cu") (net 16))
 (segment (start 187.1445 85.4584) (end 187.2461 85.4076) (width 0.1524) (layer "F.Cu") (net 14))
 (segment (start 187.1445 85.4584) (end 163.6749 85.4584) (width 0.1524) (layer "F.Cu") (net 14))
 (segment (start 133.4997 115.6336) (end 99.7461 115.6336) (width 0.1524) (layer "F.Cu") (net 14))
 (via (at 163.6749 85.4584) (size 0.7564) (drill 0.35) (layers "F.Cu" "B.Cu") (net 14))
 (via (at 133.4997 115.6336) (size 0.7564) (drill 0.35) (layers "F.Cu" "B.Cu") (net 14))
 (segment (start 163.6749 85.4584) (end 133.4997 115.6336) (width 0.1524) (layer "B.Cu") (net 14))
 (segment (start 187.2461 83.8836) (end 196.1361 92.7736) (width 0.1524) (layer "F.Cu") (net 19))
 (segment (start 196.1361 92.7736) (end 196.1361 105.8636) (width 0.1524) (layer "F.Cu") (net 19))
 (segment (start 96.9237 120.8152) (end 95.8569 121.882) (width 0.1524) (layer "F.Cu") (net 2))
 (segment (start 90.6753 88.8112) (end 103.1721 76.3144) (width 0.1524) (layer "F.Cu") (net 2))
 (segment (start 95.8569 121.882) (end 95.8569 133.1596) (width 0.1524) (layer "F.Cu") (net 2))
 (segment (start 96.3141 133.6168) (end 100.8861 133.6168) (width 0.1524) (layer "F.Cu") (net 2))
 (segment (start 100.8861 133.6168) (end 101.1909 133.312) (width 0.1524) (layer "F.Cu") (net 2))
 (segment (start 159.2553 85.1536) (end 159.1761 85.1536) (width 0.1524) (layer "F.Cu") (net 2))
 (segment (start 95.8569 133.1596) (end 96.3141 133.6168) (width 0.1524) (layer "F.Cu") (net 2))
 (segment (start 159.1029 76.3144) (end 159.2553 76.4668) (width 0.1524) (layer "F.Cu") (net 2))
 (segment (start 103.1721 76.3144) (end 159.1029 76.3144) (width 0.1524) (layer "F.Cu") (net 2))
 (segment (start 101.1909 128.8924) (end 99.3621 127.0636) (width 0.1524) (layer "F.Cu") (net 2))
 (segment (start 159.2553 76.4668) (end 159.2553 85.1536) (width 0.1524) (layer "F.Cu") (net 2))
 (segment (start 99.3621 127.0636) (end 99.3621 124.6252) (width 0.1524) (layer "F.Cu") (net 2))
 (segment (start 96.9237 120.8152) (end 96.9461 120.7136) (width 0.1524) (layer "F.Cu") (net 2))
 (segment (start 99.3621 124.6252) (end 99.2461 124.5236) (width 0.1524) (layer "F.Cu") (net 2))
 (segment (start 96.9237 120.6628) (end 90.6753 114.4144) (width 0.1524) (layer "F.Cu") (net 2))
 (segment (start 96.9237 120.6628) (end 96.9461 120.7136) (width 0.1524) (layer "F.Cu") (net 2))
 (segment (start 101.1909 133.312) (end 101.1909 128.8924) (width 0.1524) (layer "F.Cu") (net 2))
 (segment (start 90.6753 114.4144) (end 90.6753 88.8112) (width 0.1524) (layer "F.Cu") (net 2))
 (segment (start 153.3117 93.0784) (end 161.2365 85.1536) (width 0.1524) (layer "F.Cu") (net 15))
 (segment (start 138.6813 90.3352) (end 138.6561 90.2336) (width 0.1524) (layer "F.Cu") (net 15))
 (segment (start 146.9109 93.0784) (end 153.3117 93.0784) (width 0.1524) (layer "F.Cu") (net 15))
 (segment (start 144.1677 90.3352) (end 138.6813 90.3352) (width 0.1524) (layer "F.Cu") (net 15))
 (segment (start 144.1677 90.3352) (end 146.9109 93.0784) (width 0.1524) (layer "F.Cu") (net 15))
 (segment (start 161.2365 85.1536) (end 161.9761 85.1536) (width 0.1524) (layer "F.Cu") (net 15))
 (segment (start 176.9337 100.8508) (end 176.8761 100.9136) (width 0.1524) (layer "F.Cu") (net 13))
 (segment (start 180.3881 102.1208) (end 178.0833 102.1208) (width 0.1524) (layer "F.Cu") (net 13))
 (segment (start 182.1153 100.3936) (end 180.3881 102.1208) (width 0.1524) (layer "F.Cu") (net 13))
 (segment (start 176.9337 100.8508) (end 176.0193 99.9364) (width 0.1524) (layer "F.Cu") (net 13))
 (segment (start 176.8761 100.9136) (end 178.0833 102.1208) (width 0.1524) (layer "F.Cu") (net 13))
 (segment (start 97.0761 132.0928) (end 96.9461 132.1436) (width 0.1524) (layer "F.Cu") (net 13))
 (segment (start 97.0761 130.5688) (end 97.0761 132.0928) (width 0.1524) (layer "F.Cu") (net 13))
 (via (at 97.0761 130.5688) (size 0.7564) (drill 0.35) (layers "F.Cu" "B.Cu") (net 13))
 (via (at 176.0193 99.9364) (size 0.7564) (drill 0.35) (layers "F.Cu" "B.Cu") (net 13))
 (segment (start 134.8713 130.5688) (end 97.0761 130.5688) (width 0.1524) (layer "B.Cu") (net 13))
 (segment (start 176.0193 99.9364) (end 165.5037 99.9364) (width 0.1524) (layer "B.Cu") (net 13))
 (segment (start 165.5037 99.9364) (end 134.8713 130.5688) (width 0.1524) (layer "B.Cu") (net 13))
 (segment (start 191.4117 110.1472) (end 191.4117 110.1636) (width 0.1524) (layer "F.Cu") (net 8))
 (segment (start 191.4117 110.1636) (end 191.4117 130.4164) (width 0.1524) (layer "F.Cu") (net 8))
 (segment (start 191.4117 130.4164) (end 191.2593 130.5688) (width 0.1524) (layer "F.Cu") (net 8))
 (segment (start 191.4117 110.1636) (end 188.1261 110.1636) (width 0.1524) (layer "F.Cu") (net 8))
 (segment (start 184.7061 124.4728) (end 184.7061 123.2536) (width 0.1524) (layer "F.Cu") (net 8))
 (segment (start 190.8021 130.5688) (end 184.7061 124.4728) (width 0.1524) (layer "F.Cu") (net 8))
 (segment (start 184.7061 123.2536) (end 184.5761 123.2536) (width 0.1524) (layer "F.Cu") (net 8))
 (segment (start 191.2593 130.5688) (end 190.8021 130.5688) (width 0.1524) (layer "F.Cu") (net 8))
 (segment (start 196.1361 110.1636) (end 191.4117 110.1636) (width 0.1524) (layer "F.Cu") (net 8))
 (segment (start 99.2097 128.4352) (end 99.1961 128.3336) (width 0.1524) (layer "F.Cu") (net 1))
 (segment (start 100.7337 133.312) (end 100.8861 133.1596) (width 0.1524) (layer "F.Cu") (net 1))
 (segment (start 100.8861 131.1784) (end 99.2097 129.502) (width 0.1524) (layer "F.Cu") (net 1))
 (segment (start 97.9905 132.55) (end 98.7525 133.312) (width 0.1524) (layer "F.Cu") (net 1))
 (segment (start 98.7525 133.312) (end 100.7337 133.312) (width 0.1524) (layer "F.Cu") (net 1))
 (segment (start 97.9905 130.5688) (end 97.9905 132.55) (width 0.1524) (layer "F.Cu") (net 1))
 (segment (start 96.6189 125.3872) (end 96.6189 129.1972) (width 0.1524) (layer "F.Cu") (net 1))
 (segment (start 100.8861 133.1596) (end 100.8861 131.1784) (width 0.1524) (layer "F.Cu") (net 1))
 (segment (start 97.3809 124.6252) (end 96.6189 125.3872) (width 0.1524) (layer "F.Cu") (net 1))
 (segment (start 99.2097 129.502) (end 99.2097 128.4352) (width 0.1524) (layer "F.Cu") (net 1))
 (segment (start 97.3809 124.6252) (end 97.4461 124.5236) (width 0.1524) (layer "F.Cu") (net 1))
 (segment (start 96.6189 129.1972) (end 97.9905 130.5688) (width 0.1524) (layer "F.Cu") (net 1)))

